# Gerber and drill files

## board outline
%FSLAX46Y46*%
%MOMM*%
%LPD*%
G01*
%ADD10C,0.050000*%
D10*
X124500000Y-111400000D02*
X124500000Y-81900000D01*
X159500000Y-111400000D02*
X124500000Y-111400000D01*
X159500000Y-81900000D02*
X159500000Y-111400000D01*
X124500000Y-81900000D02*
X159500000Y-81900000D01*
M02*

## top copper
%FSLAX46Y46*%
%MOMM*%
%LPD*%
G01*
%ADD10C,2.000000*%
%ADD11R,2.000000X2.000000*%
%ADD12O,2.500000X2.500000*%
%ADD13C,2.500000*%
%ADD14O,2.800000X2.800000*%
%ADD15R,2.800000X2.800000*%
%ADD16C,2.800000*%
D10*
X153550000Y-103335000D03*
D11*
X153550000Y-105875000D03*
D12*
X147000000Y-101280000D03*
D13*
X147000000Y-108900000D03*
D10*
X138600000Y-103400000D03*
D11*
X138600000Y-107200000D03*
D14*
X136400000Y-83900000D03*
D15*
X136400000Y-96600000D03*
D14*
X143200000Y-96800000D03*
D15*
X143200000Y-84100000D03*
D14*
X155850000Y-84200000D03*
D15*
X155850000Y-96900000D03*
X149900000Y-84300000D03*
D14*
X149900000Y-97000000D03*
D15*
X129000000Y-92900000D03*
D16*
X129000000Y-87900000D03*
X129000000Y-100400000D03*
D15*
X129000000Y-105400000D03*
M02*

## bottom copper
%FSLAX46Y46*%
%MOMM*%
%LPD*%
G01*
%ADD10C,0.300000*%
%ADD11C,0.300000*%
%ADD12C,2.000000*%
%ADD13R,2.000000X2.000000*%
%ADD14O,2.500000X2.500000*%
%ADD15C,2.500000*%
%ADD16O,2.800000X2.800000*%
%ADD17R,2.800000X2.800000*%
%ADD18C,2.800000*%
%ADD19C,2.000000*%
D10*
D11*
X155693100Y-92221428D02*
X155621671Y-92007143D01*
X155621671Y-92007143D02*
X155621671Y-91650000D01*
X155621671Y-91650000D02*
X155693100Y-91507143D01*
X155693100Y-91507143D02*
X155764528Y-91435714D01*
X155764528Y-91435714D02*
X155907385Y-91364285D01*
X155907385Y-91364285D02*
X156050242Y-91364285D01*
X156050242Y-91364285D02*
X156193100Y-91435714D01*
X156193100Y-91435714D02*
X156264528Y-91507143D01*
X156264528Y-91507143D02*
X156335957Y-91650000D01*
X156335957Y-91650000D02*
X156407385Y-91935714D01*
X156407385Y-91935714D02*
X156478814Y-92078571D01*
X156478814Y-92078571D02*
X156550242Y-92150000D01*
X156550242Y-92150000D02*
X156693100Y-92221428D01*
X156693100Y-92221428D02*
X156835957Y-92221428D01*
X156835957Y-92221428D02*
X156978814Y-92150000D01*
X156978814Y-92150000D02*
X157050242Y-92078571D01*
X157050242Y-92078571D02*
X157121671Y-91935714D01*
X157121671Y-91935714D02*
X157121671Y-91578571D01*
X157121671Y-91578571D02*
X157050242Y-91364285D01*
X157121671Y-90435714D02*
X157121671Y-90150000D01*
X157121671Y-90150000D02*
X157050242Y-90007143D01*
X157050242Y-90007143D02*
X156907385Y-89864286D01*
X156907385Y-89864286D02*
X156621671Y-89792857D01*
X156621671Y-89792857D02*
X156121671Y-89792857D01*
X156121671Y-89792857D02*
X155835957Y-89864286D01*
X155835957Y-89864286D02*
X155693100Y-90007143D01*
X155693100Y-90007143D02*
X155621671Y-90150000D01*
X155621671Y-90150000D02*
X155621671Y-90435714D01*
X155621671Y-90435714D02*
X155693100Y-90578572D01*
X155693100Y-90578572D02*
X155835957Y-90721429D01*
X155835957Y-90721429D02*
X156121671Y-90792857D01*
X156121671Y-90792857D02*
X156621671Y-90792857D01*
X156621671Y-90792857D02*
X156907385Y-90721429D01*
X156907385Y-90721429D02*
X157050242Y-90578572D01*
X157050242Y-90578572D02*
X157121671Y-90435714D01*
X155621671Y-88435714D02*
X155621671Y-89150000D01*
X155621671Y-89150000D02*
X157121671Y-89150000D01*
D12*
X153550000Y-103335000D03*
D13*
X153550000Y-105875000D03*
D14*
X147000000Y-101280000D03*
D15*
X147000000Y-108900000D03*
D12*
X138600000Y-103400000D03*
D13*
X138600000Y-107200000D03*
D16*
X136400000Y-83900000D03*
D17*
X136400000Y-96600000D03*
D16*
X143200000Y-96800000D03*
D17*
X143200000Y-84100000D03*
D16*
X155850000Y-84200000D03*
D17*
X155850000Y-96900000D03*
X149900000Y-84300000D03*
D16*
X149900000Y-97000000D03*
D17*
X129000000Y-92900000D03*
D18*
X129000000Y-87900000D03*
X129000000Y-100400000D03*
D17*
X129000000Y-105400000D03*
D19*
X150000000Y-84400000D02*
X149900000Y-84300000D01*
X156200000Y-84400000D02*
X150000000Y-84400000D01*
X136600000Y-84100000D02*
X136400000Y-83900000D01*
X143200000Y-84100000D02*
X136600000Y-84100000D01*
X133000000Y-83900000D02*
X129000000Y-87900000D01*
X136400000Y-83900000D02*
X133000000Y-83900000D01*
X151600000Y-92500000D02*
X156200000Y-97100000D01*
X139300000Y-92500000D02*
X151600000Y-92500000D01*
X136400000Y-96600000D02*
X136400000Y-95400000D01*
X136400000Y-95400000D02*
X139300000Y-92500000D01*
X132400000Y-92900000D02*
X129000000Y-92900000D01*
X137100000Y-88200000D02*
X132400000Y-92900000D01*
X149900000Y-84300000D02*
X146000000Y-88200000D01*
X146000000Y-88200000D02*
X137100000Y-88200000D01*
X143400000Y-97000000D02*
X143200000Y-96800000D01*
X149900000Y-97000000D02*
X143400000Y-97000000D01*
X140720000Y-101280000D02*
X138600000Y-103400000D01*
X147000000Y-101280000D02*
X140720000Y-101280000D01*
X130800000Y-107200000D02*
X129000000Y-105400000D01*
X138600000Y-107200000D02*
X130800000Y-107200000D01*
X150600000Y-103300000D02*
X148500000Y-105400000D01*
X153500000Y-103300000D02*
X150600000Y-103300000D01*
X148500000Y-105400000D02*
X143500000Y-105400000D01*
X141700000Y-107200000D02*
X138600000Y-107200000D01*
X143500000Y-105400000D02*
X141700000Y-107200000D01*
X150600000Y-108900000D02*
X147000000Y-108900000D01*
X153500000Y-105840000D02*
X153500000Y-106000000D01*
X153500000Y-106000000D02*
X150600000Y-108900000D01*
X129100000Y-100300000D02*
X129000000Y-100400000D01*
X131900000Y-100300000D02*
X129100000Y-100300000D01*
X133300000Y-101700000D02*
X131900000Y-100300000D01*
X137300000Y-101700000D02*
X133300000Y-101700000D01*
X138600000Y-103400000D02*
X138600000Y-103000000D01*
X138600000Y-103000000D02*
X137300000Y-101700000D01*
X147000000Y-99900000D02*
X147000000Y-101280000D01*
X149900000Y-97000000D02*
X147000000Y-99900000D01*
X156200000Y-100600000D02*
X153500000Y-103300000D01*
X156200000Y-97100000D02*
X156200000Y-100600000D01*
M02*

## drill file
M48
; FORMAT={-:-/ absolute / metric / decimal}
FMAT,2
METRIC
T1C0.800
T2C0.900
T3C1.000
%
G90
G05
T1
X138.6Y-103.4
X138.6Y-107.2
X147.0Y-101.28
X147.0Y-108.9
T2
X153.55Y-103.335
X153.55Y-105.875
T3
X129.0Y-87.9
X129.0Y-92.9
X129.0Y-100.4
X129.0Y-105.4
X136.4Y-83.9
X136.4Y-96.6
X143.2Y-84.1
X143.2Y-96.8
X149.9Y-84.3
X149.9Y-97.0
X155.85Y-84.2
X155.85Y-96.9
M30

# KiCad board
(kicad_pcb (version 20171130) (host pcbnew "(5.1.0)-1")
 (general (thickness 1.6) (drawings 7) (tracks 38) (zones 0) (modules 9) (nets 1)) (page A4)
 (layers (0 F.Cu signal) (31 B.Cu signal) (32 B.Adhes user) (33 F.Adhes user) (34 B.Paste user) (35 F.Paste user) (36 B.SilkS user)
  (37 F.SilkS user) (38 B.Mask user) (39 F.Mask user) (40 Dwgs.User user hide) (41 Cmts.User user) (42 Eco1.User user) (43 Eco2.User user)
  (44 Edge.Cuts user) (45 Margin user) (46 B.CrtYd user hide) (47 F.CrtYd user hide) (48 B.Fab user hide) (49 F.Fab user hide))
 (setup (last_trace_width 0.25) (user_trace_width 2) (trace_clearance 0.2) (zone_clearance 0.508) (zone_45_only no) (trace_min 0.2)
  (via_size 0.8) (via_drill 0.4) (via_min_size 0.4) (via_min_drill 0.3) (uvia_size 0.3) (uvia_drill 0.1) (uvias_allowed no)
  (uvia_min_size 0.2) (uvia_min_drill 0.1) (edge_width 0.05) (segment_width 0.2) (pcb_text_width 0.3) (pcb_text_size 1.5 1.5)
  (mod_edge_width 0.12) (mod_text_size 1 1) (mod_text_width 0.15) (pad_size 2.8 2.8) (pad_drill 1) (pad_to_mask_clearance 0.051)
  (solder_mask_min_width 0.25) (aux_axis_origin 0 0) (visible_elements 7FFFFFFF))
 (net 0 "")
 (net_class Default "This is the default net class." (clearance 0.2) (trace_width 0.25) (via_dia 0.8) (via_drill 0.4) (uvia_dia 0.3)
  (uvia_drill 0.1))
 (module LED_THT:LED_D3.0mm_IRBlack (layer F.Cu) (at 153.55 105.875 90)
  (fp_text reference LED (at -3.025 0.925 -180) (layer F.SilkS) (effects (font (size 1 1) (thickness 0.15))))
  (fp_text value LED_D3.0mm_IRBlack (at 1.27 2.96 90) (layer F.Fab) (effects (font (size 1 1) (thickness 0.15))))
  (pad 2 thru_hole circle (at 2.54 0 90) (size 2 2) (drill 0.9) (layers *.Cu *.Mask))
  (pad 1 thru_hole rect (at 0 0 90) (size 2 2) (drill 0.9) (layers *.Cu *.Mask)))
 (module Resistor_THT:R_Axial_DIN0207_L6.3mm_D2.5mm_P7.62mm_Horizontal (layer F.Cu) (at 147 108.9 90)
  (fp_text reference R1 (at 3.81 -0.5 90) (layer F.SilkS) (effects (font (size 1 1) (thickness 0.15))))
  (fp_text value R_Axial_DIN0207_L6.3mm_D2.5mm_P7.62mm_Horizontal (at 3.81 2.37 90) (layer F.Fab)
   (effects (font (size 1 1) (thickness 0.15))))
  (pad 2 thru_hole oval (at 7.62 0 90) (size 2.5 2.5) (drill 0.8) (layers *.Cu *.Mask))
  (pad 1 thru_hole circle (at 0 0 90) (size 2.5 2.5) (drill 0.8) (layers *.Cu *.Mask)))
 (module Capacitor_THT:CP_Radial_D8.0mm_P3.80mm (layer F.Cu) (at 138.6 107.2 90)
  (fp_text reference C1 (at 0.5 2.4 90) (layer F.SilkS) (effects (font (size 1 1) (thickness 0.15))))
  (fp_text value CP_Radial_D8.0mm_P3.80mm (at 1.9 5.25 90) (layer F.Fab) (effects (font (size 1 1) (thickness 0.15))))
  (pad 2 thru_hole circle (at 3.8 0 90) (size 2 2) (drill 0.8) (layers *.Cu *.Mask))
  (pad 1 thru_hole rect (at 0 0 90) (size 2 2) (drill 0.8) (layers *.Cu *.Mask)))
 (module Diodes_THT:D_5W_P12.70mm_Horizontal (layer F.Cu) (at 136.4 96.6 90)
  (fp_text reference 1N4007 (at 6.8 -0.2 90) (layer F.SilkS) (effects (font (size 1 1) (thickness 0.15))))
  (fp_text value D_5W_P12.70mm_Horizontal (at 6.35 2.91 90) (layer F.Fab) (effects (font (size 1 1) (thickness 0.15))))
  (pad 2 thru_hole oval (at 12.7 0 90) (size 2.8 2.8) (drill 1) (layers *.Cu *.Mask))
  (pad 1 thru_hole rect (at 0 0 90) (size 2.8 2.8) (drill 1) (layers *.Cu *.Mask)))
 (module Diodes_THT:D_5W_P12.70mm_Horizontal (layer F.Cu) (at 143.2 84.1 270)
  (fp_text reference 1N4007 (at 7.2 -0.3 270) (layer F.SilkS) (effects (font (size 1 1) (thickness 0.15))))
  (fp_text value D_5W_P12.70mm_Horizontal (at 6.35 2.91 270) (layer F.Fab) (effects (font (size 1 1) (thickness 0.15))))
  (pad 2 thru_hole oval (at 12.7 0 270) (size 2.8 2.8) (drill 1) (layers *.Cu *.Mask))
  (pad 1 thru_hole rect (at 0 0 270) (size 2.8 2.8) (drill 1) (layers *.Cu *.Mask)))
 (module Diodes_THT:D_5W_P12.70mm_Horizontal (layer F.Cu) (at 155.85 96.9 90)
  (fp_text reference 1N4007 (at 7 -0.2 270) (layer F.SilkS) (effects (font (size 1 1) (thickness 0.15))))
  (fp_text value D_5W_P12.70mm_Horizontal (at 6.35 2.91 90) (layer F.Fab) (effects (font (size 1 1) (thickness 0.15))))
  (pad 2 thru_hole oval (at 12.7 0 90) (size 2.8 2.8) (drill 1) (layers *.Cu *.Mask))
  (pad 1 thru_hole rect (at 0 0 90) (size 2.8 2.8) (drill 1) (layers *.Cu *.Mask)))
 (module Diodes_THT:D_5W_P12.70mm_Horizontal (layer F.Cu) (at 149.9 84.3 270)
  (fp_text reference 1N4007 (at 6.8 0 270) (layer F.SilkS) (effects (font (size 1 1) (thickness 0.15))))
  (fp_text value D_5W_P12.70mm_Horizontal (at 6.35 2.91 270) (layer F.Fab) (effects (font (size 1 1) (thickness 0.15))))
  (pad 1 thru_hole rect (at 0 0 270) (size 2.8 2.8) (drill 1) (layers *.Cu *.Mask))
  (pad 2 thru_hole oval (at 12.7 0 270) (size 2.8 2.8) (drill 1) (layers *.Cu *.Mask)))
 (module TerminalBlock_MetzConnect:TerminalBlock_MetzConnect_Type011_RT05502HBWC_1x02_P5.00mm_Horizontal (layer F.Cu) (at 129 92.9 90)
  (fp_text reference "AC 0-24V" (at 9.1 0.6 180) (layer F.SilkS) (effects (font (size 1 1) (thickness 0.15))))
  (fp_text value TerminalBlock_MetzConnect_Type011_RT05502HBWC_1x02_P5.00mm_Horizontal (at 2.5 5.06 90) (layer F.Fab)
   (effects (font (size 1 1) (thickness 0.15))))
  (pad 1 thru_hole rect (at 0 0 90) (size 2.8 2.8) (drill 1) (layers *.Cu *.Mask))
  (pad 2 thru_hole circle (at 5 0 90) (size 2.8 2.8) (drill 1) (layers *.Cu *.Mask)))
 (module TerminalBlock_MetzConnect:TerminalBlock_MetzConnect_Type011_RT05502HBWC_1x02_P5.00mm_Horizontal (layer F.Cu) (at 129 105.4 90)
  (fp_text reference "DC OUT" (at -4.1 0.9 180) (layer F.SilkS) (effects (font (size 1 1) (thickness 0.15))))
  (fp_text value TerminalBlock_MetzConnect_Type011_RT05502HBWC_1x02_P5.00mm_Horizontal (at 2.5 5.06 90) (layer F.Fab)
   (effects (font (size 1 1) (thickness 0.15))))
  (pad 2 thru_hole circle (at 5 0 90) (size 2.8 2.8) (drill 1) (layers *.Cu *.Mask))
  (pad 1 thru_hole rect (at 0 0 90) (size 2.8 2.8) (drill 1) (layers *.Cu *.Mask)))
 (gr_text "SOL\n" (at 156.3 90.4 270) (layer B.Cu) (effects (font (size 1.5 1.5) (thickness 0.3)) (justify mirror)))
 (gr_line (start 124.5 111.4) (end 124.5 81.9) (layer Edge.Cuts) (width 0.05))
 (gr_line (start 159.5 111.4) (end 124.5 111.4) (layer Edge.Cuts) (width 0.05))
 (gr_line (start 159.5 81.9) (end 159.5 111.4) (layer Edge.Cuts) (width 0.05))
 (gr_line (start 124.5 81.9) (end 159.5 81.9) (layer Edge.Cuts) (width 0.05))
 (segment (start 150 84.4) (end 149.9 84.3) (width 2) (layer B.Cu) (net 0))
 (segment (start 156.2 84.4) (end 150 84.4) (width 2) (layer B.Cu) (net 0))
 (segment (start 136.6 84.1) (end 136.4 83.9) (width 2) (layer B.Cu) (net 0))
 (segment (start 143.2 84.1) (end 136.6 84.1) (width 2) (layer B.Cu) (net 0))
 (segment (start 133 83.9) (end 129 87.9) (width 2) (layer B.Cu) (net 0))
 (segment (start 136.4 83.9) (end 133 83.9) (width 2) (layer B.Cu) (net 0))
 (segment (start 151.6 92.5) (end 156.2 97.1) (width 2) (layer B.Cu) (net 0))
 (segment (start 139.3 92.5) (end 151.6 92.5) (width 2) (layer B.Cu) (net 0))
 (segment (start 136.4 96.6) (end 136.4 95.4) (width 2) (layer B.Cu) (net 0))
 (segment (start 136.4 95.4) (end 139.3 92.5) (width 2) (layer B.Cu) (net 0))
 (segment (start 132.4 92.9) (end 129 92.9) (width 2) (layer B.Cu) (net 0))
 (segment (start 137.1 88.2) (end 132.4 92.9) (width 2) (layer B.Cu) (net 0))
 (segment (start 149.9 84.3) (end 146 88.2) (width 2) (layer B.Cu) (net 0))
 (segment (start 146 88.2) (end 137.1 88.2) (width 2) (layer B.Cu) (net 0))
 (segment (start 143.4 97) (end 143.2 96.8) (width 2) (layer B.Cu) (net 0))
 (segment (start 149.9 97) (end 143.4 97) (width 2) (layer B.Cu) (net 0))
 (segment (start 140.72 101.28) (end 138.6 103.4) (width 2) (layer B.Cu) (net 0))
 (segment (start 147 101.28) (end 140.72 101.28) (width 2) (layer B.Cu) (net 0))
 (segment (start 130.8 107.2) (end 129 105.4) (width 2) (layer B.Cu) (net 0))
 (segment (start 138.6 107.2) (end 130.8 107.2) (width 2) (layer B.Cu) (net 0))
 (segment (start 150.6 103.3) (end 148.5 105.4) (width 2) (layer B.Cu) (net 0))
 (segment (start 153.5 103.3) (end 150.6 103.3) (width 2) (layer B.Cu) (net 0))
 (segment (start 148.5 105.4) (end 143.5 105.4) (width 2) (layer B.Cu) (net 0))
 (segment (start 141.7 107.2) (end 138.6 107.2) (width 2) (layer B.Cu) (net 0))
 (segment (start 143.5 105.4) (end 141.7 107.2) (width 2) (layer B.Cu) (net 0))
 (segment (start 150.6 108.9) (end 147 108.9) (width 2) (layer B.Cu) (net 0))
 (segment (start 153.5 105.84) (end 153.5 106) (width 2) (layer B.Cu) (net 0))
 (segment (start 153.5 106) (end 150.6 108.9) (width 2) (layer B.Cu) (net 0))
 (segment (start 129.1 100.3) (end 129 100.4) (width 2) (layer B.Cu) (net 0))
 (segment (start 131.9 100.3) (end 129.1 100.3) (width 2) (layer B.Cu) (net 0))
 (segment (start 133.3 101.7) (end 131.9 100.3) (width 2) (layer B.Cu) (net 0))
 (segment (start 137.3 101.7) (end 133.3 101.7) (width 2) (layer B.Cu) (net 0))
 (segment (start 138.6 103.4) (end 138.6 103) (width 2) (layer B.Cu) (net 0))
 (segment (start 138.6 103) (end 137.3 101.7) (width 2) (layer B.Cu) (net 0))
 (segment (start 147 99.9) (end 147 101.28) (width 2) (layer B.Cu) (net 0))
 (segment (start 149.9 97) (end 147 99.9) (width 2) (layer B.Cu) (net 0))
 (segment (start 156.2 100.6) (end 153.5 103.3) (width 2) (layer B.Cu) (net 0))
 (segment (start 156.2 97.1) (end 156.2 100.6) (width 2) (layer B.Cu) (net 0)))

